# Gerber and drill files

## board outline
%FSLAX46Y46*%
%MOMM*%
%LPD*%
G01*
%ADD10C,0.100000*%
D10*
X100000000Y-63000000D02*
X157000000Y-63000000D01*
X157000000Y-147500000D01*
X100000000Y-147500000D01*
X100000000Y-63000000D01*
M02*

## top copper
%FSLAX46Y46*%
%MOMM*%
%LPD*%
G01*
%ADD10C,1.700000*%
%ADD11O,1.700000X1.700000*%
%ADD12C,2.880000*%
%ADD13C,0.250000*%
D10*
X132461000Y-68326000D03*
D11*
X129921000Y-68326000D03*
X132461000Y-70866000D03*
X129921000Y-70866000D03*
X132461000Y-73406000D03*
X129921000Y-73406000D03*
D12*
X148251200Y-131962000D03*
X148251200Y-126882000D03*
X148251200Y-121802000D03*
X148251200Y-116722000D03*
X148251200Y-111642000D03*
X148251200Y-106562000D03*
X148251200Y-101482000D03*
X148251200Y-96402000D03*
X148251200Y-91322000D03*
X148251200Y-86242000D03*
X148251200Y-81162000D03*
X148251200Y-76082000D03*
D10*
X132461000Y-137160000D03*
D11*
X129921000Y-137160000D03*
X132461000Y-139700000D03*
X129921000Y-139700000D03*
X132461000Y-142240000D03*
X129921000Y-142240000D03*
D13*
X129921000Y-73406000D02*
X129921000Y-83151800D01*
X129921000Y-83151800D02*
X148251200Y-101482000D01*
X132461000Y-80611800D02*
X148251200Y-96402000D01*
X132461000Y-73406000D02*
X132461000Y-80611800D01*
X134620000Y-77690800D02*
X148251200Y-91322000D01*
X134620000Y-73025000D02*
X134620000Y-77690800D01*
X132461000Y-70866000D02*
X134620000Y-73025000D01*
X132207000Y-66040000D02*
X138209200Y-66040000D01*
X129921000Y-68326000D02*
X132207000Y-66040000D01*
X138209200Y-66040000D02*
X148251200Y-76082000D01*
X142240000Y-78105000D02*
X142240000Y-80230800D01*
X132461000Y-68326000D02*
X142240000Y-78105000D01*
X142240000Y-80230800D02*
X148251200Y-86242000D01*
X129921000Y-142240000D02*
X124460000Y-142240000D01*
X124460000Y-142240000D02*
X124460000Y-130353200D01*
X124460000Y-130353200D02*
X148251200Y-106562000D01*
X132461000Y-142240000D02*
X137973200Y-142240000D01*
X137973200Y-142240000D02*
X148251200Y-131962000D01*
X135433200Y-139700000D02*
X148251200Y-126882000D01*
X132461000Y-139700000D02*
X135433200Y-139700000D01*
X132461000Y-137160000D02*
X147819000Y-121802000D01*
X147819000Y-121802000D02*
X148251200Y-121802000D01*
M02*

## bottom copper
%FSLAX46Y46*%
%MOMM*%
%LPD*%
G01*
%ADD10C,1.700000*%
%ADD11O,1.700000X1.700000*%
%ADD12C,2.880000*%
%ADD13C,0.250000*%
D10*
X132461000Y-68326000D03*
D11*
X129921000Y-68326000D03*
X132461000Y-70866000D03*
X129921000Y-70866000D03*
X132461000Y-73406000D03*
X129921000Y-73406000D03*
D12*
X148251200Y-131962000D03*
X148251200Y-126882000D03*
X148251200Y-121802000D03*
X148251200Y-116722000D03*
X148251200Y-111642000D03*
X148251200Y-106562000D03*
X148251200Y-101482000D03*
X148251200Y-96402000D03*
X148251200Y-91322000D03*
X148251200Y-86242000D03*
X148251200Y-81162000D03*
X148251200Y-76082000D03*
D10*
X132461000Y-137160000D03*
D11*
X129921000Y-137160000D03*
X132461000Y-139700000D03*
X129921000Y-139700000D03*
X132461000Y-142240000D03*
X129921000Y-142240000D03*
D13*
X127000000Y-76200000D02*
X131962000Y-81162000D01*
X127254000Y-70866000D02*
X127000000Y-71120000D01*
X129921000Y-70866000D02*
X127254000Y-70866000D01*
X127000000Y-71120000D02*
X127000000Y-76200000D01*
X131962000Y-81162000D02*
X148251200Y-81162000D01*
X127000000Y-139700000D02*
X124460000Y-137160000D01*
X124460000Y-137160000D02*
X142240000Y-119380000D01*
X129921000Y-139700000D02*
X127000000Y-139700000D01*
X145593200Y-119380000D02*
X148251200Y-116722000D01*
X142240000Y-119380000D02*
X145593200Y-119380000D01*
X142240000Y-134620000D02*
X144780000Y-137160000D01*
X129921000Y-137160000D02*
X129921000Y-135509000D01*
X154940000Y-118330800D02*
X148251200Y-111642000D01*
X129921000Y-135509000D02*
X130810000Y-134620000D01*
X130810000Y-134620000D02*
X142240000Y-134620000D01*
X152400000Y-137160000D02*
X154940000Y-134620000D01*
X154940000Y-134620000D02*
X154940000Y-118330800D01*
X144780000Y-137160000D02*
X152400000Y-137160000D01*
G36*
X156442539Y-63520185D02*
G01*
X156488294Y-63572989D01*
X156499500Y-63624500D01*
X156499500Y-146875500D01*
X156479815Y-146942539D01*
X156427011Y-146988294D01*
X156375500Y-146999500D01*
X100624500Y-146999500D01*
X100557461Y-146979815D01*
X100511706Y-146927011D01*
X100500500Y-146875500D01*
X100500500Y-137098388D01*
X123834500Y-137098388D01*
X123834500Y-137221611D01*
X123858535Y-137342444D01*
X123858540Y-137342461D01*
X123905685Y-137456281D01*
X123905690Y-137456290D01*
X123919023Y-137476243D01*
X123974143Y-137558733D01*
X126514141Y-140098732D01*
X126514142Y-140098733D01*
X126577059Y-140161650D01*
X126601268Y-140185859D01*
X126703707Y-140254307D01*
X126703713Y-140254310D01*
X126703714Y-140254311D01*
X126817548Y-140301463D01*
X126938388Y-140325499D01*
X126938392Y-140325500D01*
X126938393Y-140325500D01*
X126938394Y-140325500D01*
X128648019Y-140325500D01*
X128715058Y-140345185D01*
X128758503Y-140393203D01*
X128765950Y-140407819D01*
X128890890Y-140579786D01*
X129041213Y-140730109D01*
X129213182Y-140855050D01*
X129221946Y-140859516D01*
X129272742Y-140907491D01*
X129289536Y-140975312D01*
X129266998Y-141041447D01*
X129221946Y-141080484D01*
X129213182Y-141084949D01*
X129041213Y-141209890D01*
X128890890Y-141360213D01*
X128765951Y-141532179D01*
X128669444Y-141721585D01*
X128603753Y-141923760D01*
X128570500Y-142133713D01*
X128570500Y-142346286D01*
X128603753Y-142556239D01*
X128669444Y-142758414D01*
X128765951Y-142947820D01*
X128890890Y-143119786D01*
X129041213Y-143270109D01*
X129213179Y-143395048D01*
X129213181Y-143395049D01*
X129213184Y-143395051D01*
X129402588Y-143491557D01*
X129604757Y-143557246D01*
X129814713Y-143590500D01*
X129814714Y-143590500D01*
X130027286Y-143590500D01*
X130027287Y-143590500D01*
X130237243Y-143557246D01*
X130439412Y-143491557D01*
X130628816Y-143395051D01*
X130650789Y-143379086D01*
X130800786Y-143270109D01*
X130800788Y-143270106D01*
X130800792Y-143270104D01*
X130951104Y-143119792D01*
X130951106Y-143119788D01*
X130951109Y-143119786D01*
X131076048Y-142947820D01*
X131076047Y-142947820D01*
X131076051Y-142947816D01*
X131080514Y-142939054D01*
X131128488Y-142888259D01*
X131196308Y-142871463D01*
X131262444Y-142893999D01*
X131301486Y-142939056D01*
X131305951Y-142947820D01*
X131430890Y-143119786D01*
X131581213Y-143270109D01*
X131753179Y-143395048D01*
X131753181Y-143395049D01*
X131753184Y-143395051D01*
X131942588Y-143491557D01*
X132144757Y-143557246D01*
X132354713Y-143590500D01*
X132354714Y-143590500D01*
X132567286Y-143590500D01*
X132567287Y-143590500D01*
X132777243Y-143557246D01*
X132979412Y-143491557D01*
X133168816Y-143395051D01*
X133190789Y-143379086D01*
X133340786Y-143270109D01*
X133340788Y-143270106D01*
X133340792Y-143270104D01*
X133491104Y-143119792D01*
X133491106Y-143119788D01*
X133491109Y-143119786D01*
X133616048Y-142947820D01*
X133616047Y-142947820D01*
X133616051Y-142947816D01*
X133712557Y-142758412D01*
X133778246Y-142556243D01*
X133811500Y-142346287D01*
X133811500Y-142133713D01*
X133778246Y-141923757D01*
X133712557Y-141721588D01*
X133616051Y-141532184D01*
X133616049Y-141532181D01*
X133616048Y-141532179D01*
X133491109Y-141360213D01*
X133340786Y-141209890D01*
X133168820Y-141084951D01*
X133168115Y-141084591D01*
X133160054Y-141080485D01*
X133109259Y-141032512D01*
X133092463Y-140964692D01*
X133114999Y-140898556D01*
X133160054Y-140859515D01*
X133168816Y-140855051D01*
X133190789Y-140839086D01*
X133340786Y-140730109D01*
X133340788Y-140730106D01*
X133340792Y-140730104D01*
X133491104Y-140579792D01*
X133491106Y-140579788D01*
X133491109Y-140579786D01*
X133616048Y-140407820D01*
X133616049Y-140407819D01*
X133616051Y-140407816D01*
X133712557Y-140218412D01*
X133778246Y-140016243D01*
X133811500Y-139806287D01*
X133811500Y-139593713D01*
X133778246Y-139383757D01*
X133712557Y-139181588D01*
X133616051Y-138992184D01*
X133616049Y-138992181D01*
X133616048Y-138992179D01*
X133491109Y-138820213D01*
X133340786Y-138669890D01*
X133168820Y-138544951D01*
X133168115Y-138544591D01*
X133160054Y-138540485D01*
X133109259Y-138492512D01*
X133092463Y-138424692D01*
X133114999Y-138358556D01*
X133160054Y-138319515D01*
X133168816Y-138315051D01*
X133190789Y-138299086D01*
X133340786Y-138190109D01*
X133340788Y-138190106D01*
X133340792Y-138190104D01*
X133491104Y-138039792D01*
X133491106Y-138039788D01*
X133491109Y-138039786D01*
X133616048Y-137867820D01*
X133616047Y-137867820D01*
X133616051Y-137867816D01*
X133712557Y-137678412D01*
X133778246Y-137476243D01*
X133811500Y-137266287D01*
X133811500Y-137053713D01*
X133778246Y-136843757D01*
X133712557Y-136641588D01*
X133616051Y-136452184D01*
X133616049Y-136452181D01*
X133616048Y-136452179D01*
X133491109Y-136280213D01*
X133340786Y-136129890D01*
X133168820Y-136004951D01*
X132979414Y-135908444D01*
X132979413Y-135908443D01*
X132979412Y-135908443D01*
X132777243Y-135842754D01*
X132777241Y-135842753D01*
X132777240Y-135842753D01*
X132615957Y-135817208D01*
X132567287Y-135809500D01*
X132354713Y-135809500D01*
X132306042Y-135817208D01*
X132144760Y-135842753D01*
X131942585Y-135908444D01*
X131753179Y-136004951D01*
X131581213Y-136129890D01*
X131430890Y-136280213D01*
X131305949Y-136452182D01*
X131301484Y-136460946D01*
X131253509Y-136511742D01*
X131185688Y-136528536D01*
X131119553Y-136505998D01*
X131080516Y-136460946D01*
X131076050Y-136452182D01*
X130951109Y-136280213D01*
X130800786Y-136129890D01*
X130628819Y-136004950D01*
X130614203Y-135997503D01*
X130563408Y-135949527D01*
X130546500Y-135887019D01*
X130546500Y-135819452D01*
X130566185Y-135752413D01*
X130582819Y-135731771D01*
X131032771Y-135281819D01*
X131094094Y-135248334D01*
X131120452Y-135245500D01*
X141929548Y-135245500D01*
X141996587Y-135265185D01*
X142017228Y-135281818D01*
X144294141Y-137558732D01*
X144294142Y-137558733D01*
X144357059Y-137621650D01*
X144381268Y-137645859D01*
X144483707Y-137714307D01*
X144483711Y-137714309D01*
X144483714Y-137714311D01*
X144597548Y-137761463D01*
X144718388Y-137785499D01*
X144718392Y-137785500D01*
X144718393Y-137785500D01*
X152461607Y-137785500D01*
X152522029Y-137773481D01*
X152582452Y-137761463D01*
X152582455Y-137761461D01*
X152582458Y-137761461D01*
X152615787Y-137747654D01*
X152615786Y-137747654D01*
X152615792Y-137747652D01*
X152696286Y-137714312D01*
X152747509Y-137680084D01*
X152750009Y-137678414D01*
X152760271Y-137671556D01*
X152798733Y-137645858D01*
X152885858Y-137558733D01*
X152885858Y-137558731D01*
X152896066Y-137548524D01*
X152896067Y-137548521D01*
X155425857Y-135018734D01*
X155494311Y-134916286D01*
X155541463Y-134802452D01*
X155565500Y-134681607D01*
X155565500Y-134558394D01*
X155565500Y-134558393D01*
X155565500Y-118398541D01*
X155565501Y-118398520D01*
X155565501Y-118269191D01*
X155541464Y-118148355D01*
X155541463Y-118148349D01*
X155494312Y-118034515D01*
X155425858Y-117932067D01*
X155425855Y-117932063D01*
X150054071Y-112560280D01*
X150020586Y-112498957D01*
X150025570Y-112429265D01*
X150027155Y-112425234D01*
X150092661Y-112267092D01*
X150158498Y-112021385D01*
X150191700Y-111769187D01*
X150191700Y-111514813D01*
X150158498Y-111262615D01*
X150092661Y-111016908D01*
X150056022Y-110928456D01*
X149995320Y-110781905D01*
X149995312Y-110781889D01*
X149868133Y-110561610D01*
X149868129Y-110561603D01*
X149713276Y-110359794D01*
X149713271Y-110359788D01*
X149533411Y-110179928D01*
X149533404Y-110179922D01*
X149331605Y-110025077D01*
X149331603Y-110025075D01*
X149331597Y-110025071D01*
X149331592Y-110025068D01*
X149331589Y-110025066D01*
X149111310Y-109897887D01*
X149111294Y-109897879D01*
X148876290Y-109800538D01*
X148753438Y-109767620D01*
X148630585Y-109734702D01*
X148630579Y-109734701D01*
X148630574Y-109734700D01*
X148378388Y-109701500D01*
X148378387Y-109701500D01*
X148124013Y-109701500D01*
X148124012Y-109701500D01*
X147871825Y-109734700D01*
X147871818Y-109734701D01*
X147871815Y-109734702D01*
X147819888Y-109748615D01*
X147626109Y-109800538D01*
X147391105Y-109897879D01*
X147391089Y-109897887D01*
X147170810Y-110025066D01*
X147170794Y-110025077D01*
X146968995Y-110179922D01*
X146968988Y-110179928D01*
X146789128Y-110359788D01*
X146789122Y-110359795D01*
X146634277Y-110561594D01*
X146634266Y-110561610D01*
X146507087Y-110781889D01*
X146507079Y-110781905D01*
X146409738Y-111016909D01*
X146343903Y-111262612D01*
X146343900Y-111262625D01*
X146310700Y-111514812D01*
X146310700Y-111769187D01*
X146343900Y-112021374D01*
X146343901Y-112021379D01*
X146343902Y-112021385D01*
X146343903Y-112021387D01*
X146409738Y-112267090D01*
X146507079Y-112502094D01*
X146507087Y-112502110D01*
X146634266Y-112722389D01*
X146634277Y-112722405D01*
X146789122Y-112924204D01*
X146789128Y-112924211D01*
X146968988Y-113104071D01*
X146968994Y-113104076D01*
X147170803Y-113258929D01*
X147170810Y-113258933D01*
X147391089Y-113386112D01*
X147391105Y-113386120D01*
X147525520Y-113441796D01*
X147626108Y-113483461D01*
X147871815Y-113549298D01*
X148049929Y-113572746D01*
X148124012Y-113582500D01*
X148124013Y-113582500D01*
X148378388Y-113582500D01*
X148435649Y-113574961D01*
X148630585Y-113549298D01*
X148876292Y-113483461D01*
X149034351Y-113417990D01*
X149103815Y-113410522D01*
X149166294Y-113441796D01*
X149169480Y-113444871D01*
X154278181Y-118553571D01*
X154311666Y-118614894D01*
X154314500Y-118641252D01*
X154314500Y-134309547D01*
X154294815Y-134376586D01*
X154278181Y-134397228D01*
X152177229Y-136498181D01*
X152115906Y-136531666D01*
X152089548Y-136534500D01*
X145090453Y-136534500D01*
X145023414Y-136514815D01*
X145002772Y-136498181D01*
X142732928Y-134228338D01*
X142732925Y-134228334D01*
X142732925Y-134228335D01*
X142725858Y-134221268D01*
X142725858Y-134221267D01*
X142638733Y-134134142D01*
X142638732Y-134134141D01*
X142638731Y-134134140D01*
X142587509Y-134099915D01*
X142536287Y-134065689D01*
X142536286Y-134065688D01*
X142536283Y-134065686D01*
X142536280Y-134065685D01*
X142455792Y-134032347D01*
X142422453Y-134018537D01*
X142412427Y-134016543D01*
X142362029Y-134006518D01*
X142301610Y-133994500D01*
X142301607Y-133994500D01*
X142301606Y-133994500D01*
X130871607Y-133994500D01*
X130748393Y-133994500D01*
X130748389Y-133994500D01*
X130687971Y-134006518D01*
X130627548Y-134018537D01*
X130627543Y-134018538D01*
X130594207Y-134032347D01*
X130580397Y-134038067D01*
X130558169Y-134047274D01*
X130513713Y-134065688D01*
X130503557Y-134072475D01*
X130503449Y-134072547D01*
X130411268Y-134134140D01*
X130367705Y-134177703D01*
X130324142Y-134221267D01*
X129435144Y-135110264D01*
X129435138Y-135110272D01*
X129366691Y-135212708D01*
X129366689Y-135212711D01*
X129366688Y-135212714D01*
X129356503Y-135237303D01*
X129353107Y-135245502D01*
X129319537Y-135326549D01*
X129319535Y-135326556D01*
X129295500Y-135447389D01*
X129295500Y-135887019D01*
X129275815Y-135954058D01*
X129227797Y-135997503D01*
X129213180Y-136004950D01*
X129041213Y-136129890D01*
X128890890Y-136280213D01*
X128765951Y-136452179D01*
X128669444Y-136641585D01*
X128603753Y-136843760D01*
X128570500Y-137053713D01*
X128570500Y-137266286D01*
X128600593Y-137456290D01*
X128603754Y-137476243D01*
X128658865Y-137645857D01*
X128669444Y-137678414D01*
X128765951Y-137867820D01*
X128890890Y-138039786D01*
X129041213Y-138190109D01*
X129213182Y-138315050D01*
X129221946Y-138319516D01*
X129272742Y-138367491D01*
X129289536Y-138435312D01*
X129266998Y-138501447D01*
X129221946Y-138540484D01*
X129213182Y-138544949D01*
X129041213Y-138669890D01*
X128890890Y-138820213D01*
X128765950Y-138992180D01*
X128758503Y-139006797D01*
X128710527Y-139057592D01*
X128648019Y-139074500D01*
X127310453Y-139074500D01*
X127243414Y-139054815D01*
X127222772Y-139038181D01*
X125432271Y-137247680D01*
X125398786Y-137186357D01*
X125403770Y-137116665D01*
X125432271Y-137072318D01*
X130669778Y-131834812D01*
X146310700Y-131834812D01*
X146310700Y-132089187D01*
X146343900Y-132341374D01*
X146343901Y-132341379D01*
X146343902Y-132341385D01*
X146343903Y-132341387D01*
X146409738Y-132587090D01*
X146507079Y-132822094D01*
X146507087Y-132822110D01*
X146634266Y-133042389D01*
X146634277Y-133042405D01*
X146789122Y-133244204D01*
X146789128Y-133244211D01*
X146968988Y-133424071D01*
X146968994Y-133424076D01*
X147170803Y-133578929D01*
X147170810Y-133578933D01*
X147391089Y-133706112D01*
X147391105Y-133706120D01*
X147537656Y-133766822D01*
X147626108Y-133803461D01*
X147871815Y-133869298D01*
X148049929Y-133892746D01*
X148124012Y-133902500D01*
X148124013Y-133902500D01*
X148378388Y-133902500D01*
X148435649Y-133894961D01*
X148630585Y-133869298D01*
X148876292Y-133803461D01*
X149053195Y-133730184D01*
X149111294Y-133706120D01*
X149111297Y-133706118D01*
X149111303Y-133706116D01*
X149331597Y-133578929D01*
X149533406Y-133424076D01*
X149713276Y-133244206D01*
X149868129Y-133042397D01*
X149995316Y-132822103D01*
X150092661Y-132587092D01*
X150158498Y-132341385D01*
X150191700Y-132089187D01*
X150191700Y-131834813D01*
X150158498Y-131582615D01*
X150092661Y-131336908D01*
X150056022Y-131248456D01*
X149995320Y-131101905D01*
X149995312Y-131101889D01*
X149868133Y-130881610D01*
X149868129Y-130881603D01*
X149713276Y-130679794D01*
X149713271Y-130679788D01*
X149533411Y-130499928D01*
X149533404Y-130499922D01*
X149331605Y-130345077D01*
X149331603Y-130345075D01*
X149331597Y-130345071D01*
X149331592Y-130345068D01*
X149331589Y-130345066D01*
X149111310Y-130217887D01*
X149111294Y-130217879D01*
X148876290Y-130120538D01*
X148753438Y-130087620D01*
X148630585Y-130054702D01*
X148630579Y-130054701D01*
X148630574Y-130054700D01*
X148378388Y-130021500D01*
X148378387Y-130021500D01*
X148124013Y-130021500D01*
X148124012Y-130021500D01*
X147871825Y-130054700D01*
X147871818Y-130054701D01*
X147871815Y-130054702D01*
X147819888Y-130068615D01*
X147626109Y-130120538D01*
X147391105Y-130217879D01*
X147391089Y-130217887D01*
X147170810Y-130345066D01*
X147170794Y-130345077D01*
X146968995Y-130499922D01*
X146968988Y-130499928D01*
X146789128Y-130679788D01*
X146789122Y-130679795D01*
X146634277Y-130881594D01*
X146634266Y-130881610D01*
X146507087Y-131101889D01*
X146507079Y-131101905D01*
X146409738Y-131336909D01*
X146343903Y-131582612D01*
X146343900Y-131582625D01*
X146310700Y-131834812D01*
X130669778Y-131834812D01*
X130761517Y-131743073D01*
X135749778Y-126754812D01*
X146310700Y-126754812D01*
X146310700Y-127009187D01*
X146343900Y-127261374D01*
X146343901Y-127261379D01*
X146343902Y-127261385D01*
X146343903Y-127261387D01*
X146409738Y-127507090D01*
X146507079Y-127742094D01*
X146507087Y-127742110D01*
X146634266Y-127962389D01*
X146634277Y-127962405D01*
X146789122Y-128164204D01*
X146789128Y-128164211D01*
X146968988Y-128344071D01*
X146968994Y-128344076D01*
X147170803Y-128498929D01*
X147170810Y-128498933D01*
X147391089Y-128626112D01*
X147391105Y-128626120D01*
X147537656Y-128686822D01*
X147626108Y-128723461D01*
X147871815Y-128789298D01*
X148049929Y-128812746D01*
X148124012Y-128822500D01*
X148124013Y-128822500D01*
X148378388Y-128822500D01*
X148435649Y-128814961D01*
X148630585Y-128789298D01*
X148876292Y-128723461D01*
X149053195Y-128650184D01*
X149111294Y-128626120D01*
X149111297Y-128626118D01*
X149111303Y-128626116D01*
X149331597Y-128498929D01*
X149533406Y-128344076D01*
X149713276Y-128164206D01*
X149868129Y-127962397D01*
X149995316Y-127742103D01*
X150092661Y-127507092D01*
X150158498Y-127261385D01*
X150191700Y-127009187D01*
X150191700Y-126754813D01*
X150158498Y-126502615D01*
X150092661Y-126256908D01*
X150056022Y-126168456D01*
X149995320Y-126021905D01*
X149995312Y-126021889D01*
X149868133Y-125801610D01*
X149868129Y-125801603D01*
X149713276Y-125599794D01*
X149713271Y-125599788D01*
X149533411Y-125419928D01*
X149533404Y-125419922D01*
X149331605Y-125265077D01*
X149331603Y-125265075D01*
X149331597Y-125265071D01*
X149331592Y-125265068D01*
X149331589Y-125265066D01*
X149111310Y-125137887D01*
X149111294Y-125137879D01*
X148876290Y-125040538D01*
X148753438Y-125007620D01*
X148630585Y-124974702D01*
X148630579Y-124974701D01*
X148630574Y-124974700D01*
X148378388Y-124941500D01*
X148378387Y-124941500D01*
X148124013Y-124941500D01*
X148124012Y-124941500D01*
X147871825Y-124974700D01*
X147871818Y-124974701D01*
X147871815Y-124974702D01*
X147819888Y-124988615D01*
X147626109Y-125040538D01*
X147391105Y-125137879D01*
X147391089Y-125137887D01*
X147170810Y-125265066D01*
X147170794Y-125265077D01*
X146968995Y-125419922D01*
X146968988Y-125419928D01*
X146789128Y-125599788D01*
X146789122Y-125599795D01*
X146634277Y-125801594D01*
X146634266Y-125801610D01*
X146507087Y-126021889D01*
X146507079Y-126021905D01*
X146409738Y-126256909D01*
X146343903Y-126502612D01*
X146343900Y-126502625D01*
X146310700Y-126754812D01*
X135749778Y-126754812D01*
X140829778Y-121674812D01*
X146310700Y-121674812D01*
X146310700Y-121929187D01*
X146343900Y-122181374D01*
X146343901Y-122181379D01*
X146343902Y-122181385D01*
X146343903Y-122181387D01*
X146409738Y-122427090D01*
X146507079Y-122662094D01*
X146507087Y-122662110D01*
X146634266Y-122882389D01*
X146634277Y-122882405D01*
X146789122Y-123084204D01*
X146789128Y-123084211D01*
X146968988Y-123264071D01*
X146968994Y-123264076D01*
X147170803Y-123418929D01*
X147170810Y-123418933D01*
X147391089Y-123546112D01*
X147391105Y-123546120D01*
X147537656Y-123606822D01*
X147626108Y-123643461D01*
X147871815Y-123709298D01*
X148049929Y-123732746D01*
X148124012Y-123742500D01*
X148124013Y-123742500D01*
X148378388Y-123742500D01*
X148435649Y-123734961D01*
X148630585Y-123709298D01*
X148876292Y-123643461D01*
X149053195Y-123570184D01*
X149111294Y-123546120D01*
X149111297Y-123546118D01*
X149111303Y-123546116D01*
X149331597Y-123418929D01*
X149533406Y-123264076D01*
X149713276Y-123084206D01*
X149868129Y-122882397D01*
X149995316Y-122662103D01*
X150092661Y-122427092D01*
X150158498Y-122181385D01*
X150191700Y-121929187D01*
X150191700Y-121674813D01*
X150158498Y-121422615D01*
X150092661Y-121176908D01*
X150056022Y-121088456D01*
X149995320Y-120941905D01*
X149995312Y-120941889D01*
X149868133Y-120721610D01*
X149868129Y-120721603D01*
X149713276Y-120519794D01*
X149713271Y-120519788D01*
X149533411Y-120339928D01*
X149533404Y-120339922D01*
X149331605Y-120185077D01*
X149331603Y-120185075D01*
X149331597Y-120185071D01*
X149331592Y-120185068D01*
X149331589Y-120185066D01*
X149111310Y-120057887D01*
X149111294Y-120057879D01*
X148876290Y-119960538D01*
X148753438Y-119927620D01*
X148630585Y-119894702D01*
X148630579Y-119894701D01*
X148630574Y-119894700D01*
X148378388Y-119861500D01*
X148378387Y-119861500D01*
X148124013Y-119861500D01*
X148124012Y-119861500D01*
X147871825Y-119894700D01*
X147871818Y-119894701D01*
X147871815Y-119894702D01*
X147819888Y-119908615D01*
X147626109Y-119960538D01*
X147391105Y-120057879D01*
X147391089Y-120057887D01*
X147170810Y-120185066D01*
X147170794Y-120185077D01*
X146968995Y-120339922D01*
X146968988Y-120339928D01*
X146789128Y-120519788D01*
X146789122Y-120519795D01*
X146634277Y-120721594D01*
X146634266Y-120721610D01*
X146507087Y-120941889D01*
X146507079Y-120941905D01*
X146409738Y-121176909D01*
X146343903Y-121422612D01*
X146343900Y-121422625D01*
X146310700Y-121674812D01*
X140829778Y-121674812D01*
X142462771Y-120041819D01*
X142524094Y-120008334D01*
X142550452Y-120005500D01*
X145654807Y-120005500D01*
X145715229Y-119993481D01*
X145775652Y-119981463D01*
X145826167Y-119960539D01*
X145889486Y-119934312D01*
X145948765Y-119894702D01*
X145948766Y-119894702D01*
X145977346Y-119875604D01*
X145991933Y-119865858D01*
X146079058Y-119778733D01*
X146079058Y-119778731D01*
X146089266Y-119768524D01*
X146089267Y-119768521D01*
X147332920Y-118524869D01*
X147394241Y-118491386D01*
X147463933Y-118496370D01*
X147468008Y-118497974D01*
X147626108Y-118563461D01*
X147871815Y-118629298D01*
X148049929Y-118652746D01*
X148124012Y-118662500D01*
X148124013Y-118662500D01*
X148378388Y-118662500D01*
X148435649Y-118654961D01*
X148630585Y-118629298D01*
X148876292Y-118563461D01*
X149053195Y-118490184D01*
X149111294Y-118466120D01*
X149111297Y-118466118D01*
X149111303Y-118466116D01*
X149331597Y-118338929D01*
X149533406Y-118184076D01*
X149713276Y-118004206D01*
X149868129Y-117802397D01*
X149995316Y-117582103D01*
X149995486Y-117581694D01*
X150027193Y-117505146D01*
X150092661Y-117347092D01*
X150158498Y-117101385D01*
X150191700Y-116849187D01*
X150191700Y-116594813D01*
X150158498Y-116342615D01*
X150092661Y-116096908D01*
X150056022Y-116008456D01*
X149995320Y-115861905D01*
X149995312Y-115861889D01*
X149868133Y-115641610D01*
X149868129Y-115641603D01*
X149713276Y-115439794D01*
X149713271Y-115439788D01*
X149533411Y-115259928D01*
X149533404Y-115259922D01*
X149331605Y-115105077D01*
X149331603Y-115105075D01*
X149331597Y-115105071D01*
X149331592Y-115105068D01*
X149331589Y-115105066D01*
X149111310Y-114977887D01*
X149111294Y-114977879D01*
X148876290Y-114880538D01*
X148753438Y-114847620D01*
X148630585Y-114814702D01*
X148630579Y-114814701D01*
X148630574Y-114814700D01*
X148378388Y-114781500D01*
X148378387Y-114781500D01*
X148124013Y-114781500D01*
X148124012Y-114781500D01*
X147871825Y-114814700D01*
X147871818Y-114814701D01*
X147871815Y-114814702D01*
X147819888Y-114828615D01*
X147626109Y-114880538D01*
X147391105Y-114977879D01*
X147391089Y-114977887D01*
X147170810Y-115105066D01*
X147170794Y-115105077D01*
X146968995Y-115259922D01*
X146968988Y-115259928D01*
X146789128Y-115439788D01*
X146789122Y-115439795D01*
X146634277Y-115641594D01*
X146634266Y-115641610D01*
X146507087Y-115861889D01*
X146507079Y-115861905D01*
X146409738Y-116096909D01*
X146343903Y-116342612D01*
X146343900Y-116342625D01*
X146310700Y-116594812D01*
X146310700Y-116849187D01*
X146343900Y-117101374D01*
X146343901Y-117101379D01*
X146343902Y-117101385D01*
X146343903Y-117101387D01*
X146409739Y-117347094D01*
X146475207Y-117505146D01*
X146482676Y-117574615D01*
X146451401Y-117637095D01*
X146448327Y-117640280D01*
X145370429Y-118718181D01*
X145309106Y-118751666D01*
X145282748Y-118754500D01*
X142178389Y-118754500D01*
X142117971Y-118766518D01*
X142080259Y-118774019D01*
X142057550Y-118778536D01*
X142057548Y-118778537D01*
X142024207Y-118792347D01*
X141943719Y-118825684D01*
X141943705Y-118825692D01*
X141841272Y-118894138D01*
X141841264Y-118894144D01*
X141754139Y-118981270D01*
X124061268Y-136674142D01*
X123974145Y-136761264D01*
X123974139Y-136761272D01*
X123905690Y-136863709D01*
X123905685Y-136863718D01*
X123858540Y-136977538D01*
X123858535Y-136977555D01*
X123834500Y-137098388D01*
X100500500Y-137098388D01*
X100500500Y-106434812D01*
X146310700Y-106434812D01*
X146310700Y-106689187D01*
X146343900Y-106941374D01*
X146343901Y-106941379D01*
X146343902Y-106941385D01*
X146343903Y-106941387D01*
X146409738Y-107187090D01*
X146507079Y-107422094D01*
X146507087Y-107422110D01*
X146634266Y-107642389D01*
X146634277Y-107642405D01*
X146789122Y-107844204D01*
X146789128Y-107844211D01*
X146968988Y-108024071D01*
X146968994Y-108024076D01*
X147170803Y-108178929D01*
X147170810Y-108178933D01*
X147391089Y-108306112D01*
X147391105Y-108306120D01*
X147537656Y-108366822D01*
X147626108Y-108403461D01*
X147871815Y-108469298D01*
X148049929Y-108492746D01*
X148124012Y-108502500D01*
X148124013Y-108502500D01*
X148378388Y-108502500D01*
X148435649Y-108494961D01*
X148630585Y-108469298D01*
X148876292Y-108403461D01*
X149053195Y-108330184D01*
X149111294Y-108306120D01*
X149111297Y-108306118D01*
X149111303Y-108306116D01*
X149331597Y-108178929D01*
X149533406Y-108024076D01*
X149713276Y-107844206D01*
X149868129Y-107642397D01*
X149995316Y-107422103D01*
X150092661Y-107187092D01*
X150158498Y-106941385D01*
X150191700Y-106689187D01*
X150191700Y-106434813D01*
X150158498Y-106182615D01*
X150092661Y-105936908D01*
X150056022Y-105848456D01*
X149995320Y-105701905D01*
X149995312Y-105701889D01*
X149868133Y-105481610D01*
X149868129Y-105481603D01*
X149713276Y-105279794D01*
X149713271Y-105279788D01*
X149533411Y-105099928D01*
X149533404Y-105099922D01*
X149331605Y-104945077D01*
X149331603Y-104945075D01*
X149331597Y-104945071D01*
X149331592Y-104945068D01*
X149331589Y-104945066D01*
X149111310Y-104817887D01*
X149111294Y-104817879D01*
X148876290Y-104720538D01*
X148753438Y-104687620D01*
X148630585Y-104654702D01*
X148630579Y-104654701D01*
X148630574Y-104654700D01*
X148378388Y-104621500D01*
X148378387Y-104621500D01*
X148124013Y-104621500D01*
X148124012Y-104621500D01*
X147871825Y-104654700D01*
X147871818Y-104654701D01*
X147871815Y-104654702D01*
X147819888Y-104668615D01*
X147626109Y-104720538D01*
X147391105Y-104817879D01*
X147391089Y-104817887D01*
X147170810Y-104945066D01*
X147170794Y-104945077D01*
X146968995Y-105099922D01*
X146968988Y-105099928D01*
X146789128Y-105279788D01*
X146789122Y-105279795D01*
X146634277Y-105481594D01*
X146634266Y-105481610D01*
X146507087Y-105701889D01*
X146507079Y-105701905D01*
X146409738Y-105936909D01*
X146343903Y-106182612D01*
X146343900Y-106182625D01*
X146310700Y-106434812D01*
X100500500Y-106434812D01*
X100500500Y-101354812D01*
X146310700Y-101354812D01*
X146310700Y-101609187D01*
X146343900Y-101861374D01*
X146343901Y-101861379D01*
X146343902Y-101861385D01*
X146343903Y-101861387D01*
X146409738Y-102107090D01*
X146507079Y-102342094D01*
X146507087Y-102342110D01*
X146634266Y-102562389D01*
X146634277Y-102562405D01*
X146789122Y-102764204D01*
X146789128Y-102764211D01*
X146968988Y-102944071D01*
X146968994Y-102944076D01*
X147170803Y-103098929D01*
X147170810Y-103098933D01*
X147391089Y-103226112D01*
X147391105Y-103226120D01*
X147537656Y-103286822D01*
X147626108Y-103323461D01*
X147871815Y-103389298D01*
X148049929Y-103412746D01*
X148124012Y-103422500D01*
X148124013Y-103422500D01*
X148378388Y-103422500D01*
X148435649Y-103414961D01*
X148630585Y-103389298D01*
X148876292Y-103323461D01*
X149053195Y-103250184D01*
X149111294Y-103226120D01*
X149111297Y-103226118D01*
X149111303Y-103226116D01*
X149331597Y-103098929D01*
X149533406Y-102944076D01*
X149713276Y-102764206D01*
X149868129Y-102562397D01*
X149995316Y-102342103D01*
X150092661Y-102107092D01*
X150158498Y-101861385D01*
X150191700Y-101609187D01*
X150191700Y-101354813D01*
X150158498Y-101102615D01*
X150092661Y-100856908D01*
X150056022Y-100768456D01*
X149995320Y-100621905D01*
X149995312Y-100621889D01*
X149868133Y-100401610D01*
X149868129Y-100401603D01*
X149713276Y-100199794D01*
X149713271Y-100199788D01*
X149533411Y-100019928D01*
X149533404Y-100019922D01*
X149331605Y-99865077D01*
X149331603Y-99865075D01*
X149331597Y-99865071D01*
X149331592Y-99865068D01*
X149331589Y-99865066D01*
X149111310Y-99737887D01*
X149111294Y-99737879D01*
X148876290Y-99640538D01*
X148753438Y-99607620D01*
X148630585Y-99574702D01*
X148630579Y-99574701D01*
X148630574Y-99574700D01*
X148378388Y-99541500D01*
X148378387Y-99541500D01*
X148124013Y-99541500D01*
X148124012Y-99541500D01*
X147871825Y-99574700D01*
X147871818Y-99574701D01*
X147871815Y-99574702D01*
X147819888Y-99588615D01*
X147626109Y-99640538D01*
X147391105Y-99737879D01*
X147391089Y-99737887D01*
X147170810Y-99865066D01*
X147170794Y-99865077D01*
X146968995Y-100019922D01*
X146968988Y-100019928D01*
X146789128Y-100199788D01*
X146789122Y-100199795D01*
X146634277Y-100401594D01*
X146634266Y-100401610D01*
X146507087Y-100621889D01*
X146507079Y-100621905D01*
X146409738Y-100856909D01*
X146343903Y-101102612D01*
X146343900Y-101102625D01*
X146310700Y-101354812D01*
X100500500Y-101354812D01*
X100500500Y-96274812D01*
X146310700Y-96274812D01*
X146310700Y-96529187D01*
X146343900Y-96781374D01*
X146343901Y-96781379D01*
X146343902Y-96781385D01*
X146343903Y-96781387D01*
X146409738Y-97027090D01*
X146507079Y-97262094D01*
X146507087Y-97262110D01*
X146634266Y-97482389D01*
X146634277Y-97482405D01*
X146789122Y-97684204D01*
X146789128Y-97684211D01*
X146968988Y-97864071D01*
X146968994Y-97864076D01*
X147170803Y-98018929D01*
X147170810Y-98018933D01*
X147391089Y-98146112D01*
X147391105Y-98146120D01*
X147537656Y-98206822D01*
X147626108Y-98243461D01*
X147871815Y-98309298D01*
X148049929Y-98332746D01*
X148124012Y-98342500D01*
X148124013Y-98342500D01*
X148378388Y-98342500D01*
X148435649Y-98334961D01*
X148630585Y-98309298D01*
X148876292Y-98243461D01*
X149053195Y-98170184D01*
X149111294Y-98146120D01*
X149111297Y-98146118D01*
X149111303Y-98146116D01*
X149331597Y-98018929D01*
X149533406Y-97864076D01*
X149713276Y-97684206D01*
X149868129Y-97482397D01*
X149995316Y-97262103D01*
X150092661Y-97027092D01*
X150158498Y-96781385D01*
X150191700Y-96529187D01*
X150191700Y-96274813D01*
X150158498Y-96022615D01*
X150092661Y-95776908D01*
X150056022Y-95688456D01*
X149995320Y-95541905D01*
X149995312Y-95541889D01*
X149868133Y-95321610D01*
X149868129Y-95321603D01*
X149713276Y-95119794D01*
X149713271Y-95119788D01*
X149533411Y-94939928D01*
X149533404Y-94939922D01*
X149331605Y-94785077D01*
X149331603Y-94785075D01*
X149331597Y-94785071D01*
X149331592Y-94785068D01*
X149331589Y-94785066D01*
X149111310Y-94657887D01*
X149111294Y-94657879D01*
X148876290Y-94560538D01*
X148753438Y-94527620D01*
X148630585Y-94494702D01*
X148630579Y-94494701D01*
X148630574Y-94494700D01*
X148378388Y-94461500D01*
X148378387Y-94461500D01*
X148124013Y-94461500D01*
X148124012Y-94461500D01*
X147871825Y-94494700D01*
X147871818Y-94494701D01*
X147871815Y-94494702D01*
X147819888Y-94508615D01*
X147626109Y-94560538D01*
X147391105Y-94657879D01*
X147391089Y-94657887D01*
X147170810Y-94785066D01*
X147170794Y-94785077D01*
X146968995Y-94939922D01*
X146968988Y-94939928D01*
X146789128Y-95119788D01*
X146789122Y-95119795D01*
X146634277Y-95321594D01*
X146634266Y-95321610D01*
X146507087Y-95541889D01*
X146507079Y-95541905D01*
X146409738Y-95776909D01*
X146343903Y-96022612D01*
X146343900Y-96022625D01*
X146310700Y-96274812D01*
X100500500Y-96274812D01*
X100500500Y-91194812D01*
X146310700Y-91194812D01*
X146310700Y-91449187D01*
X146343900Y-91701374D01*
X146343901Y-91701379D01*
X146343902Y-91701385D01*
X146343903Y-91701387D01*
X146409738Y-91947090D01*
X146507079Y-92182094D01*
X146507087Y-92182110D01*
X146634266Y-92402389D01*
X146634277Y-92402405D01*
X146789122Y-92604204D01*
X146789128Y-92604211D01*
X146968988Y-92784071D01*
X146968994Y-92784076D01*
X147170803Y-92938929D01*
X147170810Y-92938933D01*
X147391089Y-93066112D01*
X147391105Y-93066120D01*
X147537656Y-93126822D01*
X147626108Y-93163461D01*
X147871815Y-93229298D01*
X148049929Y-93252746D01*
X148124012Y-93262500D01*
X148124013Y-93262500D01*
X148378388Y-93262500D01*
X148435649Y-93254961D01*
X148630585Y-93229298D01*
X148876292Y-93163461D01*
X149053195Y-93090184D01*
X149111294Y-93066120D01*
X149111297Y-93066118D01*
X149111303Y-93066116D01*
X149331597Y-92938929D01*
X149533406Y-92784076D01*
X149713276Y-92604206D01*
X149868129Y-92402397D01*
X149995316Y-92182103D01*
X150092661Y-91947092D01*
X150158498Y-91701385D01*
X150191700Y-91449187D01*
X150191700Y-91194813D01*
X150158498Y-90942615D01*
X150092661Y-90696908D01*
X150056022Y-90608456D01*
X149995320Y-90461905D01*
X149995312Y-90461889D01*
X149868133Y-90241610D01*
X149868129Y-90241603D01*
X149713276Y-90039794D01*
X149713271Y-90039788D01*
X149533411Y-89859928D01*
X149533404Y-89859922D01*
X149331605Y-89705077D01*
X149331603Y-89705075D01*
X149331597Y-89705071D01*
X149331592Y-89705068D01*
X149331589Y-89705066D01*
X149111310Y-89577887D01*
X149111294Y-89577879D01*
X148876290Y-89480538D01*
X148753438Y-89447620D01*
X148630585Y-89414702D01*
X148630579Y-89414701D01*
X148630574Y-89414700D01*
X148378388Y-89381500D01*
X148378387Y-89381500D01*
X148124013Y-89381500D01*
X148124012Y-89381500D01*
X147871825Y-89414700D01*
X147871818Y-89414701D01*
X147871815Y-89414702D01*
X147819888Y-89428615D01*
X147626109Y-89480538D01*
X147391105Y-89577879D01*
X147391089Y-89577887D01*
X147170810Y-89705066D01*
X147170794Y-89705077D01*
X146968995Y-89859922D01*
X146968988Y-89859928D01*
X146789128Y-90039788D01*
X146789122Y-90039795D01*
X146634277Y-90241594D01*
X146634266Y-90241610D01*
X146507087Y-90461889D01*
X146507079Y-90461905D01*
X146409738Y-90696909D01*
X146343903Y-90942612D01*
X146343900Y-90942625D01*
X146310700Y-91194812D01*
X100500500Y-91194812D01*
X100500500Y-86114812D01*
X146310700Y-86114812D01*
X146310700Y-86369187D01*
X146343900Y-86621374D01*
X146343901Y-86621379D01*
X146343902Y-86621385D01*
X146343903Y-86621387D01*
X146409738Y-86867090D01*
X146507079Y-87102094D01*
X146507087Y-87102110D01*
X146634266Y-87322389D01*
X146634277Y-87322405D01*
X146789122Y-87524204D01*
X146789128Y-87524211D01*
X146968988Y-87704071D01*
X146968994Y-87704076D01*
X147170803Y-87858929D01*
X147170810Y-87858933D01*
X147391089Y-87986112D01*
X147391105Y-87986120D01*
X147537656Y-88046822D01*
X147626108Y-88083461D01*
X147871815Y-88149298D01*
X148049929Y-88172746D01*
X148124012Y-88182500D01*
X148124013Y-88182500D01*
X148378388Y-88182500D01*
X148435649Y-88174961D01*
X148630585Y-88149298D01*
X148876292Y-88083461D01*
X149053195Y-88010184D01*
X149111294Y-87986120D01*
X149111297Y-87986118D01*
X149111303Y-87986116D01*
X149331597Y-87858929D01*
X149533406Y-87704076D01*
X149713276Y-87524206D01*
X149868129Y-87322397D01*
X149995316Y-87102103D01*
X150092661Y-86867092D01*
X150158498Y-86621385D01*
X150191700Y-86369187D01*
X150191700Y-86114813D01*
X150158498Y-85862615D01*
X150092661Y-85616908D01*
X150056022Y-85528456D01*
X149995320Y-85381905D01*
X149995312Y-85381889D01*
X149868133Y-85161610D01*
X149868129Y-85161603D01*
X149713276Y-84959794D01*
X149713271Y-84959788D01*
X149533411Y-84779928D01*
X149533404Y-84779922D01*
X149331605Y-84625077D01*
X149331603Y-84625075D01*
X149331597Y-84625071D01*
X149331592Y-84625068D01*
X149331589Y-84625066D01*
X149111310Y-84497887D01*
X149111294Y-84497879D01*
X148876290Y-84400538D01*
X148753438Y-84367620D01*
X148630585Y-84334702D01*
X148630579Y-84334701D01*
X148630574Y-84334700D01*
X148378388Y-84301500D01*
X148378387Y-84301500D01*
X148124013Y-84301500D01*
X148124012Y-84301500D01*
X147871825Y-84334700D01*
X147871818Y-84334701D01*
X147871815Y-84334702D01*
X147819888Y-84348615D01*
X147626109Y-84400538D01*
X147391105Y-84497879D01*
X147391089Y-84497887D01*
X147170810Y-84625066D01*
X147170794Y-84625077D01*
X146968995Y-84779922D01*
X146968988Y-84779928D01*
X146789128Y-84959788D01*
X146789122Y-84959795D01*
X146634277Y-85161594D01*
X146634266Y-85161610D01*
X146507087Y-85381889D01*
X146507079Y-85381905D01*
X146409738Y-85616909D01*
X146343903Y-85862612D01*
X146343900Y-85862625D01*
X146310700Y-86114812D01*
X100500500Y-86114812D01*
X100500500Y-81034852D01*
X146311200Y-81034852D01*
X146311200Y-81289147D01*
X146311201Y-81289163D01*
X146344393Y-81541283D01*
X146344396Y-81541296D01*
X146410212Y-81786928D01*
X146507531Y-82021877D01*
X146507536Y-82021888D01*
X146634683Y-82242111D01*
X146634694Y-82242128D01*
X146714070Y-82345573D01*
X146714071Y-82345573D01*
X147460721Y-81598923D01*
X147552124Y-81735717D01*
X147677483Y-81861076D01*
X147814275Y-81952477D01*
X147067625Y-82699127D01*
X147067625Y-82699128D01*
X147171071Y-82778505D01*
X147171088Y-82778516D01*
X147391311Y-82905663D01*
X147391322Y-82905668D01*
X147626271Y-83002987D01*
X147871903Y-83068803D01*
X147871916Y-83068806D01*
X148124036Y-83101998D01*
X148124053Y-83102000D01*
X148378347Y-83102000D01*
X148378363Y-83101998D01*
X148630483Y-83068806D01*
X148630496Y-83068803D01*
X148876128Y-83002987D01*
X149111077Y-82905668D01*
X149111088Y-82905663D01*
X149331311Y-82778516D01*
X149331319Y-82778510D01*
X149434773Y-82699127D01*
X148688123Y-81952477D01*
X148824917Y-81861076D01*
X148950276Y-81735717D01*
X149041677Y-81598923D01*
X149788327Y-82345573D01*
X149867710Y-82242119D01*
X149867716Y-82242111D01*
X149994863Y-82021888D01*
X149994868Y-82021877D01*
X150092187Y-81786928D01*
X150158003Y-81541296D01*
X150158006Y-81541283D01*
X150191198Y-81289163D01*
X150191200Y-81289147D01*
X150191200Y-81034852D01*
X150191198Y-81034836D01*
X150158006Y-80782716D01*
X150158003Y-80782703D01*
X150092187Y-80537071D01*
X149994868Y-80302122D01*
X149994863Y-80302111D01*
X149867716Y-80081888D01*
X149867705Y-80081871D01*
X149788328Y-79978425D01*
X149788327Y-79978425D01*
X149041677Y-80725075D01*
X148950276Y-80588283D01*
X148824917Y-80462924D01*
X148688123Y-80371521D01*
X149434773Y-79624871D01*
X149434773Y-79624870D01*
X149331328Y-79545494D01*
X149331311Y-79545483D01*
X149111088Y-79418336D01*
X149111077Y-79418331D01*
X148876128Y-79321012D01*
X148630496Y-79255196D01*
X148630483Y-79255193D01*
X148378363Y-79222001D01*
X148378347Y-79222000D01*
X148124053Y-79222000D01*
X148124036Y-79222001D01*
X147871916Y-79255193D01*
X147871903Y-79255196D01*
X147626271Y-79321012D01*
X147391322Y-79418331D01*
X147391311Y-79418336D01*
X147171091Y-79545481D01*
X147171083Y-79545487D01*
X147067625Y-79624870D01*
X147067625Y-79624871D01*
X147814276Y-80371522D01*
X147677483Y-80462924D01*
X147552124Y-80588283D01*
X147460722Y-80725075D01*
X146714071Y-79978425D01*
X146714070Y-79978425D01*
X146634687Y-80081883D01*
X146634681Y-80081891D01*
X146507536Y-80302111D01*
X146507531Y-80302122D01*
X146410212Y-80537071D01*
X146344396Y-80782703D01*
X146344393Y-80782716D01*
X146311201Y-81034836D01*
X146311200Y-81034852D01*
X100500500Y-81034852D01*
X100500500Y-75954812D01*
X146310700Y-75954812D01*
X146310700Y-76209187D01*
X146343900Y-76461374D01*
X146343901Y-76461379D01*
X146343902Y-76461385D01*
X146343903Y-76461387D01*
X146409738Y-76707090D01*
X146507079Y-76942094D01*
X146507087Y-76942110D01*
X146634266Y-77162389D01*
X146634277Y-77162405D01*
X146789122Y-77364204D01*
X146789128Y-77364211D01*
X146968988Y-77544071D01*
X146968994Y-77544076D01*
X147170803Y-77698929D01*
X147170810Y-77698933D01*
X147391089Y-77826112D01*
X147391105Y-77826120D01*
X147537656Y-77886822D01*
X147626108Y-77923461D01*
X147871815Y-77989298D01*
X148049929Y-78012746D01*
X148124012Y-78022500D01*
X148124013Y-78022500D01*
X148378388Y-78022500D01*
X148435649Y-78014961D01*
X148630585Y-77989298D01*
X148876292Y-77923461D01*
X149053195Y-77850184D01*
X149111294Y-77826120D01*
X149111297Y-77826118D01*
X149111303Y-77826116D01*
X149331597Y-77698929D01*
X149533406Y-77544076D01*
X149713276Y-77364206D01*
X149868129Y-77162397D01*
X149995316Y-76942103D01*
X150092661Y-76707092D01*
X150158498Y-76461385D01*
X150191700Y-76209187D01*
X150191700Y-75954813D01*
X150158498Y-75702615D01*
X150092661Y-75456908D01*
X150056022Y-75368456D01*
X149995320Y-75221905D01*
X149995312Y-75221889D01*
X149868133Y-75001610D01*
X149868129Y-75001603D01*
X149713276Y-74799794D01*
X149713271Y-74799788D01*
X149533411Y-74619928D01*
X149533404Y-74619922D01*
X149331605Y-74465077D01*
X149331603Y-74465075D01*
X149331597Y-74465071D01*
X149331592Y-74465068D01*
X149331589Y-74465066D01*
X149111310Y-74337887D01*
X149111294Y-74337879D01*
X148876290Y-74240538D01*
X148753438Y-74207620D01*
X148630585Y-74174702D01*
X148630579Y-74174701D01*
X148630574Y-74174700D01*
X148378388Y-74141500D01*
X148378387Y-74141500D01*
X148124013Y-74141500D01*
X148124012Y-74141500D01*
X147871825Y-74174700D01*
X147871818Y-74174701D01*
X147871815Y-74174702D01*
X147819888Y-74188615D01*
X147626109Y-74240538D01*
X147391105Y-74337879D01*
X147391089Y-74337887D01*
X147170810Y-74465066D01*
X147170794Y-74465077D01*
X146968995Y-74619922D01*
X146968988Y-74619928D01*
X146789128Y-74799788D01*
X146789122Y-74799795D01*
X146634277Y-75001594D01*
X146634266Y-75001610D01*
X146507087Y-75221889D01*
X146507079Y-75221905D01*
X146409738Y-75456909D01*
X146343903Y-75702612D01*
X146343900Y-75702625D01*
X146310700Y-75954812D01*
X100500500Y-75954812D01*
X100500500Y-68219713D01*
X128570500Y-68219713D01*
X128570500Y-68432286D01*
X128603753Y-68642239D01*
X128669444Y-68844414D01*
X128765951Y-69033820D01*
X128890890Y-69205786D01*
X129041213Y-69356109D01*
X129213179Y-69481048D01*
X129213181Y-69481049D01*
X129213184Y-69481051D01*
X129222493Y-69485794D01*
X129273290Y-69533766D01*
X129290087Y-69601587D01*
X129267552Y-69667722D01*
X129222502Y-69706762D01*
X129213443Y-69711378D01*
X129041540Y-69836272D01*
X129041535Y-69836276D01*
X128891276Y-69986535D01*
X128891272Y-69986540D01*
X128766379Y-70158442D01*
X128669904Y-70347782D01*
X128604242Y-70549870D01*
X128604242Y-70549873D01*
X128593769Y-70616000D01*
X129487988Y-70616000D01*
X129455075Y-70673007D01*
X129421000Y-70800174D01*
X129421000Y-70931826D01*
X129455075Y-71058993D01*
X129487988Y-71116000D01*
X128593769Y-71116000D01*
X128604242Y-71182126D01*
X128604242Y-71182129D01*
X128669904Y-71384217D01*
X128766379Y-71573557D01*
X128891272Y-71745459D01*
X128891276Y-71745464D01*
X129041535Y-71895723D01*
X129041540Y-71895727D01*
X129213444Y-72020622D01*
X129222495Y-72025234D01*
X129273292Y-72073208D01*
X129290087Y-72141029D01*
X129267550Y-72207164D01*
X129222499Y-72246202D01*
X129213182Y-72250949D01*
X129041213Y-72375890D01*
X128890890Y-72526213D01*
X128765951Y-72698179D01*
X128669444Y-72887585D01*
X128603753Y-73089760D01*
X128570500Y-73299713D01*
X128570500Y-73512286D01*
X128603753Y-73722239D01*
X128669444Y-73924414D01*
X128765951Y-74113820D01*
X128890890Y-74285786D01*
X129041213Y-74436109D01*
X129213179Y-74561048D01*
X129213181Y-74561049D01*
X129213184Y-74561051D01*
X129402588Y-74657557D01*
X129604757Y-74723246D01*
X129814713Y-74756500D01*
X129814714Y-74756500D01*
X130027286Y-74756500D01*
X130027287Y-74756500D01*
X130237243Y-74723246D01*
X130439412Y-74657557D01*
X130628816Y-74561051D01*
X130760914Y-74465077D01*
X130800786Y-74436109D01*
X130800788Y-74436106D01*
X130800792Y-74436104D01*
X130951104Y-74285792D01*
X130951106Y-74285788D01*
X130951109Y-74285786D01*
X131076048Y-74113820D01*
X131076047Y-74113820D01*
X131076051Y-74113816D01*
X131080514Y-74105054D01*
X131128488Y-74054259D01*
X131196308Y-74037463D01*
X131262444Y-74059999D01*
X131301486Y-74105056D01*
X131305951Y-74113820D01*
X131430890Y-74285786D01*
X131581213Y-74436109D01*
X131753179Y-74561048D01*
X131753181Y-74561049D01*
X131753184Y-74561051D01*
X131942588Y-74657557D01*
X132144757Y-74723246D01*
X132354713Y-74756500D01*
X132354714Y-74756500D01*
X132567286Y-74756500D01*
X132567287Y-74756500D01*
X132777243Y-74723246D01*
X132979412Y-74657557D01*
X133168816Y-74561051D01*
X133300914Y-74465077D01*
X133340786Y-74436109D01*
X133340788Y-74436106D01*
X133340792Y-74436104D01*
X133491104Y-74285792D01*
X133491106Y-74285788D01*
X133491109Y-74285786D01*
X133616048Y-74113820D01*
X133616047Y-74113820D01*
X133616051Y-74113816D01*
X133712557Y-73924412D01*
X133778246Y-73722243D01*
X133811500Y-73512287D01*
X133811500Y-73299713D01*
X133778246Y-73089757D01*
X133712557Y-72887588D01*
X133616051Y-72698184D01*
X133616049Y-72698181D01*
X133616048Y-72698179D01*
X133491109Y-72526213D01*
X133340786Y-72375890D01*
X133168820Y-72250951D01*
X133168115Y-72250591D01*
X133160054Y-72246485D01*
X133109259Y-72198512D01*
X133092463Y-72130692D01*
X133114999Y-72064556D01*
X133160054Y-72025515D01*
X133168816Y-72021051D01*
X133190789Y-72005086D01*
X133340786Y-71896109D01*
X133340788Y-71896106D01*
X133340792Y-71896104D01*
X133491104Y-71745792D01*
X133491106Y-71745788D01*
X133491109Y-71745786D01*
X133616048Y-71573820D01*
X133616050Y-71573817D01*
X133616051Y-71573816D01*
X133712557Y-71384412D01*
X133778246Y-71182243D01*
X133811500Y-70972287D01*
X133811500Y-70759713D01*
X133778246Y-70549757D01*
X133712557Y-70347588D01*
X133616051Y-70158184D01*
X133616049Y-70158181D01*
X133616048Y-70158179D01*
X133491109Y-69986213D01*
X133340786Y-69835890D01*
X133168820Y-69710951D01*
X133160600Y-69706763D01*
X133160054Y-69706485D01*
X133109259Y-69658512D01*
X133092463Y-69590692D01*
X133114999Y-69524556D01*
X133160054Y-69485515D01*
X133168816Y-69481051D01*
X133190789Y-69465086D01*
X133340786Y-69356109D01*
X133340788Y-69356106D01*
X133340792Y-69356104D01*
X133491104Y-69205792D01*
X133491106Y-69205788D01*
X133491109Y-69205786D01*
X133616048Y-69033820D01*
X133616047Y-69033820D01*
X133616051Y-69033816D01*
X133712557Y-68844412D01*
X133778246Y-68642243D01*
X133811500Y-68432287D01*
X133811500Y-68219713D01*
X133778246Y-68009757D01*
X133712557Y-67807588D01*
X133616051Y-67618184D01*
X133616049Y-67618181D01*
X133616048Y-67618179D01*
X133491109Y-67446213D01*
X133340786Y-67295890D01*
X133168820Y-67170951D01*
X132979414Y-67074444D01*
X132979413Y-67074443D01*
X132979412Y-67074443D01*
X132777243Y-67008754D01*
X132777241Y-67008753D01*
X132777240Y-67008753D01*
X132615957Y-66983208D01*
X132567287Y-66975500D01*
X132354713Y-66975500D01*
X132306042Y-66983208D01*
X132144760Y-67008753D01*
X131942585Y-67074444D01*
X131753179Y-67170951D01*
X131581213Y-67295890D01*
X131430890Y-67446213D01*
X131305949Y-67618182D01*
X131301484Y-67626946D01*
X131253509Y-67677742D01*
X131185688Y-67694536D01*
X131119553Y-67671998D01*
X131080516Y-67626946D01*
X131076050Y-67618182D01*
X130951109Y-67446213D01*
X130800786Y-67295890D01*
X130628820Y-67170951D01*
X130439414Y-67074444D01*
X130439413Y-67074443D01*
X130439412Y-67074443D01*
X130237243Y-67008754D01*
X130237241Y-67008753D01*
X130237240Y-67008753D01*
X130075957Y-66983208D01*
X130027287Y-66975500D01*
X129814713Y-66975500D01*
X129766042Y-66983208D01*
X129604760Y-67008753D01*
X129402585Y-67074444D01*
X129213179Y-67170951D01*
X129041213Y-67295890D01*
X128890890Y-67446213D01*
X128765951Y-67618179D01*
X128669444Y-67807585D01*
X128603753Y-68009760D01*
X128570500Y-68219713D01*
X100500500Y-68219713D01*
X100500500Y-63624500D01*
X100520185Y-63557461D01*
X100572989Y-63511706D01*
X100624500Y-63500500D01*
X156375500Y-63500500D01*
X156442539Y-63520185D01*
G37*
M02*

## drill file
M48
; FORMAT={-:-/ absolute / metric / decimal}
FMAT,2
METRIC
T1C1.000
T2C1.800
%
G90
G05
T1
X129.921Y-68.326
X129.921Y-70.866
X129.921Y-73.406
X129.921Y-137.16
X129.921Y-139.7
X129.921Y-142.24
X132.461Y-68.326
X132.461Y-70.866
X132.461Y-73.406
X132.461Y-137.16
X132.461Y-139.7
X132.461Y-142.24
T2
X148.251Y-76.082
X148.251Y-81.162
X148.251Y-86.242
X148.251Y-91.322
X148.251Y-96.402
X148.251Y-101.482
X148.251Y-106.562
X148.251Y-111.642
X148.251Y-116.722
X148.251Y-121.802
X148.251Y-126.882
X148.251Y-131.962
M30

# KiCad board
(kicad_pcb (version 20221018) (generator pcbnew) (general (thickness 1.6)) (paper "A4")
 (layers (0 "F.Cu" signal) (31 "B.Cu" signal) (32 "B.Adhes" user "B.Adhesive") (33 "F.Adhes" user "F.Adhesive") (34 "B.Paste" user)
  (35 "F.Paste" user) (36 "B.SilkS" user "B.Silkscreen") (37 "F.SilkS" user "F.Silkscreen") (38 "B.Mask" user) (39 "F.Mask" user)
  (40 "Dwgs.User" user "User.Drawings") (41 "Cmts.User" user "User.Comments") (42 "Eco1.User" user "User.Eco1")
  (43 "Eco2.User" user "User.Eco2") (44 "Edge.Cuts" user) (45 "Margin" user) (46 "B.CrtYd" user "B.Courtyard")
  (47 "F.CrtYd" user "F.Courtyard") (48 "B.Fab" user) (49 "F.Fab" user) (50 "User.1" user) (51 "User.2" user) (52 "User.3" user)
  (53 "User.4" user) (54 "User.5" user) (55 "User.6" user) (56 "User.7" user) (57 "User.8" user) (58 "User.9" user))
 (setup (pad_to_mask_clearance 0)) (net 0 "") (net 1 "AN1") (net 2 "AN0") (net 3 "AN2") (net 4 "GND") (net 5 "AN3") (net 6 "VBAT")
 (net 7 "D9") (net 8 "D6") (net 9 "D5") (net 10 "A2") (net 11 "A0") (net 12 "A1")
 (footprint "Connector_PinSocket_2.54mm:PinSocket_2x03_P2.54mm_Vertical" (layer "F.Cu") (at 132.461 68.326)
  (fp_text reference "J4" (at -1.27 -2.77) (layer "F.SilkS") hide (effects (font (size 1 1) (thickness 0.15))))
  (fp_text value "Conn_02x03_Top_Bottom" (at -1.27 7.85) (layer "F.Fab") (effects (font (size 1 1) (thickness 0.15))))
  (pad "1" thru_hole circle (at 0 0) (size 1.7 1.7) (drill 1) (layers "*.Cu" "*.Mask") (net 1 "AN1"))
  (pad "2" thru_hole oval (at -2.54 0) (size 1.7 1.7) (drill 1) (layers "*.Cu" "*.Mask") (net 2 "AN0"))
  (pad "3" thru_hole oval (at 0 2.54) (size 1.7 1.7) (drill 1) (layers "*.Cu" "*.Mask") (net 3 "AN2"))
  (pad "4" thru_hole oval (at -2.54 2.54) (size 1.7 1.7) (drill 1) (layers "*.Cu" "*.Mask") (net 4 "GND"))
  (pad "5" thru_hole oval (at 0 5.08) (size 1.7 1.7) (drill 1) (layers "*.Cu" "*.Mask") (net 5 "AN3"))
  (pad "6" thru_hole oval (at -2.54 5.08) (size 1.7 1.7) (drill 1) (layers "*.Cu" "*.Mask") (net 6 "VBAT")))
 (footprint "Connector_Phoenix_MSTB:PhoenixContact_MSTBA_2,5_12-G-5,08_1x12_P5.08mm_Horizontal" (layer "F.Cu") (at 148.2512 131.962 90)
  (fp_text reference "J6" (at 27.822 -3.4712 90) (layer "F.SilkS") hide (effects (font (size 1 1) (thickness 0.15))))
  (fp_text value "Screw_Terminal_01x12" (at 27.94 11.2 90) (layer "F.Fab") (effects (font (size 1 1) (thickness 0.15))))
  (pad "1" thru_hole circle (at 0 0 90) (size 2.88 2.88) (drill 1.8) (layers "*.Cu" "*.Mask") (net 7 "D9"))
  (pad "2" thru_hole circle (at 5.08 0 90) (size 2.88 2.88) (drill 1.8) (layers "*.Cu" "*.Mask") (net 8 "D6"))
  (pad "3" thru_hole circle (at 10.16 0 90) (size 2.88 2.88) (drill 1.8) (layers "*.Cu" "*.Mask") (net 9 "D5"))
  (pad "4" thru_hole circle (at 15.24 0 90) (size 2.88 2.88) (drill 1.8) (layers "*.Cu" "*.Mask") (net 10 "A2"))
  (pad "5" thru_hole circle (at 20.32 0 90) (size 2.88 2.88) (drill 1.8) (layers "*.Cu" "*.Mask") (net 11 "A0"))
  (pad "6" thru_hole circle (at 25.4 0 90) (size 2.88 2.88) (drill 1.8) (layers "*.Cu" "*.Mask") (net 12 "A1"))
  (pad "7" thru_hole circle (at 30.48 0 90) (size 2.88 2.88) (drill 1.8) (layers "*.Cu" "*.Mask") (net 6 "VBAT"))
  (pad "8" thru_hole circle (at 35.56 0 90) (size 2.88 2.88) (drill 1.8) (layers "*.Cu" "*.Mask") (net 5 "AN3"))
  (pad "9" thru_hole circle (at 40.64 0 90) (size 2.88 2.88) (drill 1.8) (layers "*.Cu" "*.Mask") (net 3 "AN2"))
  (pad "10" thru_hole circle (at 45.72 0 90) (size 2.88 2.88) (drill 1.8) (layers "*.Cu" "*.Mask") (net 1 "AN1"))
  (pad "11" thru_hole circle (at 50.8 0 90) (size 2.88 2.88) (drill 1.8) (layers "*.Cu" "*.Mask") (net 4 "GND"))
  (pad "12" thru_hole circle (at 55.88 0 90) (size 2.88 2.88) (drill 1.8) (layers "*.Cu" "*.Mask") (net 2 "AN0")))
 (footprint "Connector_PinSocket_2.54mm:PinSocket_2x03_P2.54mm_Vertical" (layer "F.Cu") (at 132.461 137.16)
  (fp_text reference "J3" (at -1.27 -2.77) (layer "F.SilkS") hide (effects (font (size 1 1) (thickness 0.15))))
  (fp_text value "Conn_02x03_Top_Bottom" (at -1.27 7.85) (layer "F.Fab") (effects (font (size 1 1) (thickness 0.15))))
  (pad "1" thru_hole circle (at 0 0) (size 1.7 1.7) (drill 1) (layers "*.Cu" "*.Mask") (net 9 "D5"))
  (pad "2" thru_hole oval (at -2.54 0) (size 1.7 1.7) (drill 1) (layers "*.Cu" "*.Mask") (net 11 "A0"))
  (pad "3" thru_hole oval (at 0 2.54) (size 1.7 1.7) (drill 1) (layers "*.Cu" "*.Mask") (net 8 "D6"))
  (pad "4" thru_hole oval (at -2.54 2.54) (size 1.7 1.7) (drill 1) (layers "*.Cu" "*.Mask") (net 10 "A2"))
  (pad "5" thru_hole oval (at 0 5.08) (size 1.7 1.7) (drill 1) (layers "*.Cu" "*.Mask") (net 7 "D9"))
  (pad "6" thru_hole oval (at -2.54 5.08) (size 1.7 1.7) (drill 1) (layers "*.Cu" "*.Mask") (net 12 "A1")))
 (gr_rect (start 100 63) (end 157 147.5) (stroke (width 0.1) (type default)) (fill none) (layer "Edge.Cuts"))
 (segment (start 129.921 73.406) (end 129.921 83.1518) (width 0.25) (layer "F.Cu") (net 6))
 (segment (start 129.921 83.1518) (end 148.2512 101.482) (width 0.25) (layer "F.Cu") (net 6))
 (segment (start 132.461 80.6118) (end 148.2512 96.402) (width 0.25) (layer "F.Cu") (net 5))
 (segment (start 132.461 73.406) (end 132.461 80.6118) (width 0.25) (layer "F.Cu") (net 5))
 (segment (start 127 76.2) (end 131.962 81.162) (width 0.25) (layer "B.Cu") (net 4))
 (segment (start 127.254 70.866) (end 127 71.12) (width 0.25) (layer "B.Cu") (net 4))
 (segment (start 129.921 70.866) (end 127.254 70.866) (width 0.25) (layer "B.Cu") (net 4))
 (segment (start 127 71.12) (end 127 76.2) (width 0.25) (layer "B.Cu") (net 4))
 (segment (start 131.962 81.162) (end 148.2512 81.162) (width 0.25) (layer "B.Cu") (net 4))
 (segment (start 134.62 77.6908) (end 148.2512 91.322) (width 0.25) (layer "F.Cu") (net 3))
 (segment (start 134.62 73.025) (end 134.62 77.6908) (width 0.25) (layer "F.Cu") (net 3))
 (segment (start 132.461 70.866) (end 134.62 73.025) (width 0.25) (layer "F.Cu") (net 3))
 (segment (start 132.207 66.04) (end 138.2092 66.04) (width 0.25) (layer "F.Cu") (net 2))
 (segment (start 129.921 68.326) (end 132.207 66.04) (width 0.25) (layer "F.Cu") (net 2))
 (segment (start 138.2092 66.04) (end 148.2512 76.082) (width 0.25) (layer "F.Cu") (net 2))
 (segment (start 142.24 78.105) (end 142.24 80.2308) (width 0.25) (layer "F.Cu") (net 1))
 (segment (start 132.461 68.326) (end 142.24 78.105) (width 0.25) (layer "F.Cu") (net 1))
 (segment (start 142.24 80.2308) (end 148.2512 86.242) (width 0.25) (layer "F.Cu") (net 1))
 (segment (start 129.921 142.24) (end 124.46 142.24) (width 0.25) (layer "F.Cu") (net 12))
 (segment (start 124.46 142.24) (end 124.46 130.3532) (width 0.25) (layer "F.Cu") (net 12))
 (segment (start 124.46 130.3532) (end 148.2512 106.562) (width 0.25) (layer "F.Cu") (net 12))
 (segment (start 132.461 142.24) (end 137.9732 142.24) (width 0.25) (layer "F.Cu") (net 7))
 (segment (start 137.9732 142.24) (end 148.2512 131.962) (width 0.25) (layer "F.Cu") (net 7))
 (segment (start 127 139.7) (end 124.46 137.16) (width 0.25) (layer "B.Cu") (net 10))
 (segment (start 124.46 137.16) (end 142.24 119.38) (width 0.25) (layer "B.Cu") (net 10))
 (segment (start 129.921 139.7) (end 127 139.7) (width 0.25) (layer "B.Cu") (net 10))
 (segment (start 145.5932 119.38) (end 148.2512 116.722) (width 0.25) (layer "B.Cu") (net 10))
 (segment (start 142.24 119.38) (end 145.5932 119.38) (width 0.25) (layer "B.Cu") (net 10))
 (segment (start 135.4332 139.7) (end 148.2512 126.882) (width 0.25) (layer "F.Cu") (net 8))
 (segment (start 132.461 139.7) (end 135.4332 139.7) (width 0.25) (layer "F.Cu") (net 8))
 (segment (start 142.24 134.62) (end 144.78 137.16) (width 0.25) (layer "B.Cu") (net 11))
 (segment (start 129.921 137.16) (end 129.921 135.509) (width 0.25) (layer "B.Cu") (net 11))
 (segment (start 154.94 118.3308) (end 148.2512 111.642) (width 0.25) (layer "B.Cu") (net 11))
 (segment (start 129.921 135.509) (end 130.81 134.62) (width 0.25) (layer "B.Cu") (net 11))
 (segment (start 130.81 134.62) (end 142.24 134.62) (width 0.25) (layer "B.Cu") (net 11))
 (segment (start 152.4 137.16) (end 154.94 134.62) (width 0.25) (layer "B.Cu") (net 11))
 (segment (start 154.94 134.62) (end 154.94 118.3308) (width 0.25) (layer "B.Cu") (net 11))
 (segment (start 144.78 137.16) (end 152.4 137.16) (width 0.25) (layer "B.Cu") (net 11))
 (segment (start 132.461 137.16) (end 147.819 121.802) (width 0.25) (layer "F.Cu") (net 9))
 (segment (start 147.819 121.802) (end 148.2512 121.802) (width 0.25) (layer "F.Cu") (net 9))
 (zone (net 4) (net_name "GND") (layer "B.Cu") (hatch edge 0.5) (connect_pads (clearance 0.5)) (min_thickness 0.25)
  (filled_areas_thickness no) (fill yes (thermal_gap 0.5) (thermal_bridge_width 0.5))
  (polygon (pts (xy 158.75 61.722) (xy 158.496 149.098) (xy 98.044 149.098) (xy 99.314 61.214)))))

